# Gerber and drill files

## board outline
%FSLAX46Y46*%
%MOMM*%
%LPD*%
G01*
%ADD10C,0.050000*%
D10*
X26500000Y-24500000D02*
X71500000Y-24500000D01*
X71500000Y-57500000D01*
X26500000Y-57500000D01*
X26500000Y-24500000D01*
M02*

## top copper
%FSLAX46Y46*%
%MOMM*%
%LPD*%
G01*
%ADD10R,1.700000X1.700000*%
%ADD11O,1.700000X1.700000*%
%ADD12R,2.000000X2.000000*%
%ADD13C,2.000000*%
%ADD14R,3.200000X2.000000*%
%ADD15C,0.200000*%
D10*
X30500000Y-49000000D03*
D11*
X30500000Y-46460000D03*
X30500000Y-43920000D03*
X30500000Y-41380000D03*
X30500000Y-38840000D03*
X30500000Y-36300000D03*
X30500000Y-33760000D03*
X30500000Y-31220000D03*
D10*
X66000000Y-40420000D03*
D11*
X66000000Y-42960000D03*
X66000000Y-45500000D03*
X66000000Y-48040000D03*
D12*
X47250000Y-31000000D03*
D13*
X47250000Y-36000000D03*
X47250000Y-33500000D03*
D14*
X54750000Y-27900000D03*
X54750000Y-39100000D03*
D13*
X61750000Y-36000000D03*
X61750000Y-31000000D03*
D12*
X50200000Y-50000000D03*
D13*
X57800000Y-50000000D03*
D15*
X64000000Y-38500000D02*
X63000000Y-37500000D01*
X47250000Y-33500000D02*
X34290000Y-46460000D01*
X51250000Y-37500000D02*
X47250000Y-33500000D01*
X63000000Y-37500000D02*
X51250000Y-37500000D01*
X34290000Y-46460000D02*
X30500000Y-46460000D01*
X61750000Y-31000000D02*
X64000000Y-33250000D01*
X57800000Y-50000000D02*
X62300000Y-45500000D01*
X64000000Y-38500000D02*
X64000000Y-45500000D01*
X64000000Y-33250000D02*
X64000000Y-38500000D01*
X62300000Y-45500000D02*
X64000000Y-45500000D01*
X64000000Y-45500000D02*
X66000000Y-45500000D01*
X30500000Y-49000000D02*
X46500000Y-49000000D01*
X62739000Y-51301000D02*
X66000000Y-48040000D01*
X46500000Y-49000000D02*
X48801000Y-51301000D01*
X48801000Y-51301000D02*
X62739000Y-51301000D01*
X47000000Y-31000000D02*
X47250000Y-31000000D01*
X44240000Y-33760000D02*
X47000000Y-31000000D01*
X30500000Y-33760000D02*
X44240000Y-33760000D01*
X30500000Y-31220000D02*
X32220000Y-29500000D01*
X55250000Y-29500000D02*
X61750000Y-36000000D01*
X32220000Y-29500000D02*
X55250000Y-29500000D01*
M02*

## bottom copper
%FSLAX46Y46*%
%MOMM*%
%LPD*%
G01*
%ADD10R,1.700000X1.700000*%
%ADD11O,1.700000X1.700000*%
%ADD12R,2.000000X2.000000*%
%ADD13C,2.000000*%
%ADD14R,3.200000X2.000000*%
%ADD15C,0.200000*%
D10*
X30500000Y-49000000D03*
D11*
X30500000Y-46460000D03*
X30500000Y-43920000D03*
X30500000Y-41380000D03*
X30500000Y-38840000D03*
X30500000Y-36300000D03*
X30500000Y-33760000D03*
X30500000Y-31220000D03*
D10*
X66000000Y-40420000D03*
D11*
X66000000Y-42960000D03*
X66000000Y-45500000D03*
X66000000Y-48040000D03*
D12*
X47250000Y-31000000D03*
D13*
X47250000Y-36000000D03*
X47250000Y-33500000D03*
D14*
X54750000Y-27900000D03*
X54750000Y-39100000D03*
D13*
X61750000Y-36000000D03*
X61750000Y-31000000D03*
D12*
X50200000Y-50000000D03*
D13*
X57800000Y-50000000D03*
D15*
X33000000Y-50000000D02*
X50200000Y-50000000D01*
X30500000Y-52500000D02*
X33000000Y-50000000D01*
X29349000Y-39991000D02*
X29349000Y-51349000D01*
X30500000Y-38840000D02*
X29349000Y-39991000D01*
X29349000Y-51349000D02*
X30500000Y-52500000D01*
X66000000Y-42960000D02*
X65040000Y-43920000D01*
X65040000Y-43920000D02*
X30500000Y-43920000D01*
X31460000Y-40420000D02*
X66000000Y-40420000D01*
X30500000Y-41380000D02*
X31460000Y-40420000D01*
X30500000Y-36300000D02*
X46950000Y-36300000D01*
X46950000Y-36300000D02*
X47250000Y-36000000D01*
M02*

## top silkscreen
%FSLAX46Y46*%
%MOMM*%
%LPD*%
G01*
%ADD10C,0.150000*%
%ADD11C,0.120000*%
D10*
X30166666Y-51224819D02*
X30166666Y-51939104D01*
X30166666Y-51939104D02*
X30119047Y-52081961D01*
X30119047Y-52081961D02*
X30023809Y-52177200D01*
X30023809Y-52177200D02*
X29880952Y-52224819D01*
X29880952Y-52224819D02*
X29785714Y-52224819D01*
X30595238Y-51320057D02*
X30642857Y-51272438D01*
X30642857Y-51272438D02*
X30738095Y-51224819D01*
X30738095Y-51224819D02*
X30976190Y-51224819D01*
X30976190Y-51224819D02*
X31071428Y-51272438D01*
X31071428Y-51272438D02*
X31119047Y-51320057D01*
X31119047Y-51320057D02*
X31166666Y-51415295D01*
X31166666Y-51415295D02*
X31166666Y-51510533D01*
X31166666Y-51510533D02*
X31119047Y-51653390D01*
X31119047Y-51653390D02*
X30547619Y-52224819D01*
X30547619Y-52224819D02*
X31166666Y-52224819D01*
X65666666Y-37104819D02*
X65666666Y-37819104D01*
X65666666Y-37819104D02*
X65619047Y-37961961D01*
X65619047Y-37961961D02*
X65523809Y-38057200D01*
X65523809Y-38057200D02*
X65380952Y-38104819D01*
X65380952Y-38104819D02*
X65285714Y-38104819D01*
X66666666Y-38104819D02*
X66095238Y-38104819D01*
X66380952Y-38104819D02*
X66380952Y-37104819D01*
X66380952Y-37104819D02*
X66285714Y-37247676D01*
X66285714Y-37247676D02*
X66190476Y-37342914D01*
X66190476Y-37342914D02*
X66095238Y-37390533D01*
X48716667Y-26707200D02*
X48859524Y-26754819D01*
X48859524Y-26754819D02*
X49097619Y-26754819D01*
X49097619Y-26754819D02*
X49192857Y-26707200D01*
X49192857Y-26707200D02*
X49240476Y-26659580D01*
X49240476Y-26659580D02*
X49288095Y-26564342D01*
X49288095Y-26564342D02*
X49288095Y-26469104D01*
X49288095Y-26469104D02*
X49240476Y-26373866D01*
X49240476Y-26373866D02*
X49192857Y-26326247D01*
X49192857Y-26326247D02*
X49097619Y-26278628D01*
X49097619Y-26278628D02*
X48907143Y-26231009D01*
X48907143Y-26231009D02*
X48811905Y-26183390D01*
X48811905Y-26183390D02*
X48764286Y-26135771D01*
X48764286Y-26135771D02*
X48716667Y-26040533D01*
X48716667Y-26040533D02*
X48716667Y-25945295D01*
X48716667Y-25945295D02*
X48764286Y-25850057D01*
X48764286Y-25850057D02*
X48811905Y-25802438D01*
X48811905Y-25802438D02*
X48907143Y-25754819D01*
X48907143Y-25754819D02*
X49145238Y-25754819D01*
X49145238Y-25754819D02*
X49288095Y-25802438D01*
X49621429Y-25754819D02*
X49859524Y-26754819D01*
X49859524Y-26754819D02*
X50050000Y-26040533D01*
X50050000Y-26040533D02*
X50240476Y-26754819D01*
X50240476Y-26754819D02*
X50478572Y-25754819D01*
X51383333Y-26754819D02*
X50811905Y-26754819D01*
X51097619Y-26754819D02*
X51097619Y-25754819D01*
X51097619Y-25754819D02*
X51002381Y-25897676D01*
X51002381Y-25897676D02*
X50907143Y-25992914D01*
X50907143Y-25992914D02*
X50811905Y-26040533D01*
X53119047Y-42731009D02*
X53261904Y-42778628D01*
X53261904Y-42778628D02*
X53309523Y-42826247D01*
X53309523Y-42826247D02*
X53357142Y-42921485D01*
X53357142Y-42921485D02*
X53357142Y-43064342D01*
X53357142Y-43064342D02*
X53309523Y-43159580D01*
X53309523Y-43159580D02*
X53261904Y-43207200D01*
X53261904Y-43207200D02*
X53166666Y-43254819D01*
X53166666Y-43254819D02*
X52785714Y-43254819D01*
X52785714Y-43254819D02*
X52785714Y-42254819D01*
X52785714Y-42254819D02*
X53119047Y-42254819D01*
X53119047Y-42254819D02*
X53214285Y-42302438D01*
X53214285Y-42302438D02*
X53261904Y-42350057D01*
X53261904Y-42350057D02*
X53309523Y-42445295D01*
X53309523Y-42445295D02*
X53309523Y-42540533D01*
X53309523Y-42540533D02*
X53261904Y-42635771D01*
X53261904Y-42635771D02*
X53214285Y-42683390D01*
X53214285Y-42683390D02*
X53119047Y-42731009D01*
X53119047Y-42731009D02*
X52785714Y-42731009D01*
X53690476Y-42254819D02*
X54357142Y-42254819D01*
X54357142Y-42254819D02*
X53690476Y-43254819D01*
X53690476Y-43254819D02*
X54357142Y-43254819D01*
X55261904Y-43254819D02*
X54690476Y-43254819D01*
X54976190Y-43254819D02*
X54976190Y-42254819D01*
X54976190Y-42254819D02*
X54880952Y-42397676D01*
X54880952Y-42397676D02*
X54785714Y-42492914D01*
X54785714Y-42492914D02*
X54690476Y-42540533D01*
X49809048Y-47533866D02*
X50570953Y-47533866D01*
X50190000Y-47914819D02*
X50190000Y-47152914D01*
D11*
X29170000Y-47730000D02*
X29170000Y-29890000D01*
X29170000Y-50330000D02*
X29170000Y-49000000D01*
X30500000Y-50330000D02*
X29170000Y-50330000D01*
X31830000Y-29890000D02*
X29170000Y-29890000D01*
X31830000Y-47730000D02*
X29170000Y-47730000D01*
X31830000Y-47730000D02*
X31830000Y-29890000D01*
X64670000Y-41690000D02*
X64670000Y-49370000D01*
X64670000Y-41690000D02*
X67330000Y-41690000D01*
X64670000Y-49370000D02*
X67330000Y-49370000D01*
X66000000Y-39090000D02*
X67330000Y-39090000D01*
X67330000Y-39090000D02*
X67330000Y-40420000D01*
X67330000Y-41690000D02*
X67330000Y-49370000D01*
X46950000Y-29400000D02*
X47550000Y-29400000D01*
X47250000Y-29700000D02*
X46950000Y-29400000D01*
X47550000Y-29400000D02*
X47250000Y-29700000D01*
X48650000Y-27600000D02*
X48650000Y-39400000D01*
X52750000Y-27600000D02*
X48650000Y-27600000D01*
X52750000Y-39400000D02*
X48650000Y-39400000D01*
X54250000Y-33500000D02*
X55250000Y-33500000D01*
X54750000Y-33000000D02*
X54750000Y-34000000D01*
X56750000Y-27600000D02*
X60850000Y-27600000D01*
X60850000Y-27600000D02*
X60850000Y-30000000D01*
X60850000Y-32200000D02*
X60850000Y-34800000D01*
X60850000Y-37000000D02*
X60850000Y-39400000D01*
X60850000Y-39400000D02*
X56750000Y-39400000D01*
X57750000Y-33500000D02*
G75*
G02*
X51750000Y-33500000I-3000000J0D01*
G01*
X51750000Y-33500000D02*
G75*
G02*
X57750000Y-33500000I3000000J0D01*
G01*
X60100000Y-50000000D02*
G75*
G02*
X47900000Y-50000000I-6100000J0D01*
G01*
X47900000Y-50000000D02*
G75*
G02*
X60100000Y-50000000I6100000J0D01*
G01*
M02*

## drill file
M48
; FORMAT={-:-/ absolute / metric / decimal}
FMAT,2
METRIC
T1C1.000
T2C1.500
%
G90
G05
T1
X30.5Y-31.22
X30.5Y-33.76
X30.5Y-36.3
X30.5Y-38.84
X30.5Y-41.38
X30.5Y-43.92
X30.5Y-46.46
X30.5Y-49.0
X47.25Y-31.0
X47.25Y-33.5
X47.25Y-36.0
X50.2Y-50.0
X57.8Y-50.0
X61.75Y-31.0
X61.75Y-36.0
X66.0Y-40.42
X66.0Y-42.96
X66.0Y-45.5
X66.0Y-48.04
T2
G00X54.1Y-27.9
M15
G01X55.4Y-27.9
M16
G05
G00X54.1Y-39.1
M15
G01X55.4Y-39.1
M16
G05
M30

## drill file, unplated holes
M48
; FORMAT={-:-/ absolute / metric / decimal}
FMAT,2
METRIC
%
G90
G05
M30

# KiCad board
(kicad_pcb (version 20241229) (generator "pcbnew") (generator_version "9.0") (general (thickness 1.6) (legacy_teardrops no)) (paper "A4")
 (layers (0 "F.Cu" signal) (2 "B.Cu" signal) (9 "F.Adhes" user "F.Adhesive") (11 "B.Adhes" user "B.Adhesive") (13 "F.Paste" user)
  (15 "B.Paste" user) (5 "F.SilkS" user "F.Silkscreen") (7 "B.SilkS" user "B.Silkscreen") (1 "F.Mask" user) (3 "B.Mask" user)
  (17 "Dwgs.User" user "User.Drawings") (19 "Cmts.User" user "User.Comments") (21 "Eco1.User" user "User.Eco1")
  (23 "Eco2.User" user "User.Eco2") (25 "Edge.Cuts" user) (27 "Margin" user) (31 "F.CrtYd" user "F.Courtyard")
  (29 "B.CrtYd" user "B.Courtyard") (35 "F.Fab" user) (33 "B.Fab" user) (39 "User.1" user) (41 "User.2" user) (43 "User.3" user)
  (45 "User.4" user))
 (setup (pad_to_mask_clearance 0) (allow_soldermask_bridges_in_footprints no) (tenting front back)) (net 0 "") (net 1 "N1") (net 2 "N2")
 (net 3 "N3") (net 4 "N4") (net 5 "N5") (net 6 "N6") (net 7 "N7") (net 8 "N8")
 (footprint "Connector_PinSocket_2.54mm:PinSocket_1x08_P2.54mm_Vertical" (layer "F.Cu") (at 30.5 49 180)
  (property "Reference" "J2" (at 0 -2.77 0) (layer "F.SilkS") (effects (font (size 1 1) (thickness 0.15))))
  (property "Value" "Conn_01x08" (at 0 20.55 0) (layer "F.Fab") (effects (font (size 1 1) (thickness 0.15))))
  (fp_line (start 1.33 1.27) (end 1.33 19.11) (stroke (width 0.12) (type solid)) (layer "F.SilkS"))
  (fp_line (start 1.33 -1.33) (end 1.33 0) (stroke (width 0.12) (type solid)) (layer "F.SilkS"))
  (fp_line (start 0 -1.33) (end 1.33 -1.33) (stroke (width 0.12) (type solid)) (layer "F.SilkS"))
  (fp_line (start -1.33 19.11) (end 1.33 19.11) (stroke (width 0.12) (type solid)) (layer "F.SilkS"))
  (fp_line (start -1.33 1.27) (end 1.33 1.27) (stroke (width 0.12) (type solid)) (layer "F.SilkS"))
  (fp_line (start -1.33 1.27) (end -1.33 19.11) (stroke (width 0.12) (type solid)) (layer "F.SilkS"))
  (pad "1" thru_hole rect (at 0 0 180) (size 1.7 1.7) (drill 1) (layers "*.Cu" "*.Mask") (remove_unused_layers no) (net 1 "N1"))
  (pad "2" thru_hole oval (at 0 2.54 180) (size 1.7 1.7) (drill 1) (layers "*.Cu" "*.Mask") (remove_unused_layers no) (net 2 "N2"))
  (pad "3" thru_hole oval (at 0 5.08 180) (size 1.7 1.7) (drill 1) (layers "*.Cu" "*.Mask") (remove_unused_layers no) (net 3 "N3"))
  (pad "4" thru_hole oval (at 0 7.62 180) (size 1.7 1.7) (drill 1) (layers "*.Cu" "*.Mask") (remove_unused_layers no) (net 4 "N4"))
  (pad "5" thru_hole oval (at 0 10.16 180) (size 1.7 1.7) (drill 1) (layers "*.Cu" "*.Mask") (remove_unused_layers no) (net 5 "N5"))
  (pad "6" thru_hole oval (at 0 12.7 180) (size 1.7 1.7) (drill 1) (layers "*.Cu" "*.Mask") (remove_unused_layers no) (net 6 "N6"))
  (pad "7" thru_hole oval (at 0 15.24 180) (size 1.7 1.7) (drill 1) (layers "*.Cu" "*.Mask") (remove_unused_layers no) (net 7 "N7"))
  (pad "8" thru_hole oval (at 0 17.78 180) (size 1.7 1.7) (drill 1) (layers "*.Cu" "*.Mask") (remove_unused_layers no) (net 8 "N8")))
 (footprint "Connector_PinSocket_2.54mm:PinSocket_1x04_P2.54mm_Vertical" (layer "F.Cu") (at 66 40.42)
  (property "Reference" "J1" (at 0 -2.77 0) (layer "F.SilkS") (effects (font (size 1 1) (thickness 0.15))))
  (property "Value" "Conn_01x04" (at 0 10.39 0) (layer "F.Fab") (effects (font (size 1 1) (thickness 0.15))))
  (fp_line (start -1.33 1.27) (end -1.33 8.95) (stroke (width 0.12) (type solid)) (layer "F.SilkS"))
  (fp_line (start -1.33 1.27) (end 1.33 1.27) (stroke (width 0.12) (type solid)) (layer "F.SilkS"))
  (fp_line (start -1.33 8.95) (end 1.33 8.95) (stroke (width 0.12) (type solid)) (layer "F.SilkS"))
  (fp_line (start 0 -1.33) (end 1.33 -1.33) (stroke (width 0.12) (type solid)) (layer "F.SilkS"))
  (fp_line (start 1.33 -1.33) (end 1.33 0) (stroke (width 0.12) (type solid)) (layer "F.SilkS"))
  (fp_line (start 1.33 1.27) (end 1.33 8.95) (stroke (width 0.12) (type solid)) (layer "F.SilkS"))
  (pad "1" thru_hole rect (at 0 0) (size 1.7 1.7) (drill 1) (layers "*.Cu" "*.Mask") (remove_unused_layers no) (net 4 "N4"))
  (pad "2" thru_hole oval (at 0 2.54) (size 1.7 1.7) (drill 1) (layers "*.Cu" "*.Mask") (remove_unused_layers no) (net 3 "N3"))
  (pad "3" thru_hole oval (at 0 5.08) (size 1.7 1.7) (drill 1) (layers "*.Cu" "*.Mask") (remove_unused_layers no) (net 2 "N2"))
  (pad "4" thru_hole oval (at 0 7.62) (size 1.7 1.7) (drill 1) (layers "*.Cu" "*.Mask") (remove_unused_layers no) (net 1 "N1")))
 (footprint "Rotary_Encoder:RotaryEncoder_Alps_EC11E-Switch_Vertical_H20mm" (layer "F.Cu") (at 47.25 31)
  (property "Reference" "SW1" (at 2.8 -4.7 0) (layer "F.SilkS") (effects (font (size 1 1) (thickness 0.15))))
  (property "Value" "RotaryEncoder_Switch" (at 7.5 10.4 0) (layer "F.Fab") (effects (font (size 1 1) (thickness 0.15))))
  (fp_line (start -0.3 -1.6) (end 0.3 -1.6) (stroke (width 0.12) (type solid)) (layer "F.SilkS"))
  (fp_line (start 0 -1.3) (end -0.3 -1.6) (stroke (width 0.12) (type solid)) (layer "F.SilkS"))
  (fp_line (start 0.3 -1.6) (end 0 -1.3) (stroke (width 0.12) (type solid)) (layer "F.SilkS"))
  (fp_line (start 1.4 -3.4) (end 1.4 8.4) (stroke (width 0.12) (type solid)) (layer "F.SilkS"))
  (fp_line (start 5.5 -3.4) (end 1.4 -3.4) (stroke (width 0.12) (type solid)) (layer "F.SilkS"))
  (fp_line (start 5.5 8.4) (end 1.4 8.4) (stroke (width 0.12) (type solid)) (layer "F.SilkS"))
  (fp_line (start 7 2.5) (end 8 2.5) (stroke (width 0.12) (type solid)) (layer "F.SilkS"))
  (fp_line (start 7.5 2) (end 7.5 3) (stroke (width 0.12) (type solid)) (layer "F.SilkS"))
  (fp_line (start 9.5 -3.4) (end 13.6 -3.4) (stroke (width 0.12) (type solid)) (layer "F.SilkS"))
  (fp_line (start 13.6 -3.4) (end 13.6 -1) (stroke (width 0.12) (type solid)) (layer "F.SilkS"))
  (fp_line (start 13.6 1.2) (end 13.6 3.8) (stroke (width 0.12) (type solid)) (layer "F.SilkS"))
  (fp_line (start 13.6 6) (end 13.6 8.4) (stroke (width 0.12) (type solid)) (layer "F.SilkS"))
  (fp_line (start 13.6 8.4) (end 9.5 8.4) (stroke (width 0.12) (type solid)) (layer "F.SilkS"))
  (fp_circle (center 7.5 2.5) (end 10.5 2.5) (stroke (width 0.12) (type solid)) (fill no) (layer "F.SilkS"))
  (pad "A" thru_hole rect (at 0 0) (size 2 2) (drill 1) (layers "*.Cu" "*.Mask") (remove_unused_layers no) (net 7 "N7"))
  (pad "B" thru_hole circle (at 0 5) (size 2 2) (drill 1) (layers "*.Cu" "*.Mask") (remove_unused_layers no) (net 6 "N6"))
  (pad "C" thru_hole circle (at 0 2.5) (size 2 2) (drill 1) (layers "*.Cu" "*.Mask") (remove_unused_layers no) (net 2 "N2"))
  (pad "MP" thru_hole rect (at 7.5 -3.1) (size 3.2 2) (drill oval 2.8 1.5) (layers "*.Cu" "*.Mask") (remove_unused_layers no))
  (pad "MP" thru_hole rect (at 7.5 8.1) (size 3.2 2) (drill oval 2.8 1.5) (layers "*.Cu" "*.Mask") (remove_unused_layers no))
  (pad "S1" thru_hole circle (at 14.5 5) (size 2 2) (drill 1) (layers "*.Cu" "*.Mask") (remove_unused_layers no) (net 8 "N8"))
  (pad "S2" thru_hole circle (at 14.5 0) (size 2 2) (drill 1) (layers "*.Cu" "*.Mask") (remove_unused_layers no) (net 2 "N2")))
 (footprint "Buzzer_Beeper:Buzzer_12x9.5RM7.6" (layer "F.Cu") (at 50.2 50)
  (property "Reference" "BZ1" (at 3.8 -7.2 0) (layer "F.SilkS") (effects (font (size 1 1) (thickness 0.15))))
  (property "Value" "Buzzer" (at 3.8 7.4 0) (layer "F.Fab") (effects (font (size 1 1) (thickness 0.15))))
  (fp_circle (center 3.8 0) (end 9.9 0) (stroke (width 0.12) (type solid)) (fill no) (layer "F.SilkS"))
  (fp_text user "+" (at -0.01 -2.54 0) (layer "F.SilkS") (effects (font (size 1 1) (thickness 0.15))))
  (pad "1" thru_hole rect (at 0 0) (size 2 2) (drill 1) (layers "*.Cu" "*.Mask") (remove_unused_layers no) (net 5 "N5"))
  (pad "2" thru_hole circle (at 7.6 0) (size 2 2) (drill 1) (layers "*.Cu" "*.Mask") (remove_unused_layers no) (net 2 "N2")))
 (gr_rect (start 26.5 24.5) (end 71.5 57.5) (stroke (width 0.05) (type default)) (fill no) (layer "Edge.Cuts"))
 (segment (start 33 50) (end 50.2 50) (width 0.2) (layer "B.Cu") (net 5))
 (segment (start 30.5 52.5) (end 33 50) (width 0.2) (layer "B.Cu") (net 5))
 (segment (start 29.349 39.991) (end 29.349 51.349) (width 0.2) (layer "B.Cu") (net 5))
 (segment (start 30.5 38.84) (end 29.349 39.991) (width 0.2) (layer "B.Cu") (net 5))
 (segment (start 29.349 51.349) (end 30.5 52.5) (width 0.2) (layer "B.Cu") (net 5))
 (segment (start 64 38.5) (end 63 37.5) (width 0.2) (layer "F.Cu") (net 2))
 (segment (start 47.25 33.5) (end 34.29 46.46) (width 0.2) (layer "F.Cu") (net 2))
 (segment (start 51.25 37.5) (end 47.25 33.5) (width 0.2) (layer "F.Cu") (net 2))
 (segment (start 63 37.5) (end 51.25 37.5) (width 0.2) (layer "F.Cu") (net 2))
 (segment (start 34.29 46.46) (end 30.5 46.46) (width 0.2) (layer "F.Cu") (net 2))
 (segment (start 61.75 31) (end 64 33.25) (width 0.2) (layer "F.Cu") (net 2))
 (segment (start 57.8 50) (end 62.3 45.5) (width 0.2) (layer "F.Cu") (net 2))
 (segment (start 64 38.5) (end 64 45.5) (width 0.2) (layer "F.Cu") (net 2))
 (segment (start 64 33.25) (end 64 38.5) (width 0.2) (layer "F.Cu") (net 2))
 (segment (start 62.3 45.5) (end 64 45.5) (width 0.2) (layer "F.Cu") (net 2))
 (segment (start 64 45.5) (end 66 45.5) (width 0.2) (layer "F.Cu") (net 2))
 (segment (start 66 42.96) (end 65.04 43.92) (width 0.2) (layer "B.Cu") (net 3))
 (segment (start 65.04 43.92) (end 30.5 43.92) (width 0.2) (layer "B.Cu") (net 3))
 (segment (start 31.46 40.42) (end 66 40.42) (width 0.2) (layer "B.Cu") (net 4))
 (segment (start 30.5 41.38) (end 31.46 40.42) (width 0.2) (layer "B.Cu") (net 4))
 (segment (start 30.5 49) (end 46.5 49) (width 0.2) (layer "F.Cu") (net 1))
 (segment (start 62.739 51.301) (end 66 48.04) (width 0.2) (layer "F.Cu") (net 1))
 (segment (start 46.5 49) (end 48.801 51.301) (width 0.2) (layer "F.Cu") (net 1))
 (segment (start 48.801 51.301) (end 62.739 51.301) (width 0.2) (layer "F.Cu") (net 1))
 (segment (start 30.5 36.3) (end 46.95 36.3) (width 0.2) (layer "B.Cu") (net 6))
 (segment (start 46.95 36.3) (end 47.25 36) (width 0.2) (layer "B.Cu") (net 6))
 (segment (start 47 31) (end 47.25 31) (width 0.2) (layer "F.Cu") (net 7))
 (segment (start 44.24 33.76) (end 47 31) (width 0.2) (layer "F.Cu") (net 7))
 (segment (start 30.5 33.76) (end 44.24 33.76) (width 0.2) (layer "F.Cu") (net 7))
 (segment (start 30.5 31.22) (end 32.22 29.5) (width 0.2) (layer "F.Cu") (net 8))
 (segment (start 55.25 29.5) (end 61.75 36) (width 0.2) (layer "F.Cu") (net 8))
 (segment (start 32.22 29.5) (end 55.25 29.5) (width 0.2) (layer "F.Cu") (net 8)))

